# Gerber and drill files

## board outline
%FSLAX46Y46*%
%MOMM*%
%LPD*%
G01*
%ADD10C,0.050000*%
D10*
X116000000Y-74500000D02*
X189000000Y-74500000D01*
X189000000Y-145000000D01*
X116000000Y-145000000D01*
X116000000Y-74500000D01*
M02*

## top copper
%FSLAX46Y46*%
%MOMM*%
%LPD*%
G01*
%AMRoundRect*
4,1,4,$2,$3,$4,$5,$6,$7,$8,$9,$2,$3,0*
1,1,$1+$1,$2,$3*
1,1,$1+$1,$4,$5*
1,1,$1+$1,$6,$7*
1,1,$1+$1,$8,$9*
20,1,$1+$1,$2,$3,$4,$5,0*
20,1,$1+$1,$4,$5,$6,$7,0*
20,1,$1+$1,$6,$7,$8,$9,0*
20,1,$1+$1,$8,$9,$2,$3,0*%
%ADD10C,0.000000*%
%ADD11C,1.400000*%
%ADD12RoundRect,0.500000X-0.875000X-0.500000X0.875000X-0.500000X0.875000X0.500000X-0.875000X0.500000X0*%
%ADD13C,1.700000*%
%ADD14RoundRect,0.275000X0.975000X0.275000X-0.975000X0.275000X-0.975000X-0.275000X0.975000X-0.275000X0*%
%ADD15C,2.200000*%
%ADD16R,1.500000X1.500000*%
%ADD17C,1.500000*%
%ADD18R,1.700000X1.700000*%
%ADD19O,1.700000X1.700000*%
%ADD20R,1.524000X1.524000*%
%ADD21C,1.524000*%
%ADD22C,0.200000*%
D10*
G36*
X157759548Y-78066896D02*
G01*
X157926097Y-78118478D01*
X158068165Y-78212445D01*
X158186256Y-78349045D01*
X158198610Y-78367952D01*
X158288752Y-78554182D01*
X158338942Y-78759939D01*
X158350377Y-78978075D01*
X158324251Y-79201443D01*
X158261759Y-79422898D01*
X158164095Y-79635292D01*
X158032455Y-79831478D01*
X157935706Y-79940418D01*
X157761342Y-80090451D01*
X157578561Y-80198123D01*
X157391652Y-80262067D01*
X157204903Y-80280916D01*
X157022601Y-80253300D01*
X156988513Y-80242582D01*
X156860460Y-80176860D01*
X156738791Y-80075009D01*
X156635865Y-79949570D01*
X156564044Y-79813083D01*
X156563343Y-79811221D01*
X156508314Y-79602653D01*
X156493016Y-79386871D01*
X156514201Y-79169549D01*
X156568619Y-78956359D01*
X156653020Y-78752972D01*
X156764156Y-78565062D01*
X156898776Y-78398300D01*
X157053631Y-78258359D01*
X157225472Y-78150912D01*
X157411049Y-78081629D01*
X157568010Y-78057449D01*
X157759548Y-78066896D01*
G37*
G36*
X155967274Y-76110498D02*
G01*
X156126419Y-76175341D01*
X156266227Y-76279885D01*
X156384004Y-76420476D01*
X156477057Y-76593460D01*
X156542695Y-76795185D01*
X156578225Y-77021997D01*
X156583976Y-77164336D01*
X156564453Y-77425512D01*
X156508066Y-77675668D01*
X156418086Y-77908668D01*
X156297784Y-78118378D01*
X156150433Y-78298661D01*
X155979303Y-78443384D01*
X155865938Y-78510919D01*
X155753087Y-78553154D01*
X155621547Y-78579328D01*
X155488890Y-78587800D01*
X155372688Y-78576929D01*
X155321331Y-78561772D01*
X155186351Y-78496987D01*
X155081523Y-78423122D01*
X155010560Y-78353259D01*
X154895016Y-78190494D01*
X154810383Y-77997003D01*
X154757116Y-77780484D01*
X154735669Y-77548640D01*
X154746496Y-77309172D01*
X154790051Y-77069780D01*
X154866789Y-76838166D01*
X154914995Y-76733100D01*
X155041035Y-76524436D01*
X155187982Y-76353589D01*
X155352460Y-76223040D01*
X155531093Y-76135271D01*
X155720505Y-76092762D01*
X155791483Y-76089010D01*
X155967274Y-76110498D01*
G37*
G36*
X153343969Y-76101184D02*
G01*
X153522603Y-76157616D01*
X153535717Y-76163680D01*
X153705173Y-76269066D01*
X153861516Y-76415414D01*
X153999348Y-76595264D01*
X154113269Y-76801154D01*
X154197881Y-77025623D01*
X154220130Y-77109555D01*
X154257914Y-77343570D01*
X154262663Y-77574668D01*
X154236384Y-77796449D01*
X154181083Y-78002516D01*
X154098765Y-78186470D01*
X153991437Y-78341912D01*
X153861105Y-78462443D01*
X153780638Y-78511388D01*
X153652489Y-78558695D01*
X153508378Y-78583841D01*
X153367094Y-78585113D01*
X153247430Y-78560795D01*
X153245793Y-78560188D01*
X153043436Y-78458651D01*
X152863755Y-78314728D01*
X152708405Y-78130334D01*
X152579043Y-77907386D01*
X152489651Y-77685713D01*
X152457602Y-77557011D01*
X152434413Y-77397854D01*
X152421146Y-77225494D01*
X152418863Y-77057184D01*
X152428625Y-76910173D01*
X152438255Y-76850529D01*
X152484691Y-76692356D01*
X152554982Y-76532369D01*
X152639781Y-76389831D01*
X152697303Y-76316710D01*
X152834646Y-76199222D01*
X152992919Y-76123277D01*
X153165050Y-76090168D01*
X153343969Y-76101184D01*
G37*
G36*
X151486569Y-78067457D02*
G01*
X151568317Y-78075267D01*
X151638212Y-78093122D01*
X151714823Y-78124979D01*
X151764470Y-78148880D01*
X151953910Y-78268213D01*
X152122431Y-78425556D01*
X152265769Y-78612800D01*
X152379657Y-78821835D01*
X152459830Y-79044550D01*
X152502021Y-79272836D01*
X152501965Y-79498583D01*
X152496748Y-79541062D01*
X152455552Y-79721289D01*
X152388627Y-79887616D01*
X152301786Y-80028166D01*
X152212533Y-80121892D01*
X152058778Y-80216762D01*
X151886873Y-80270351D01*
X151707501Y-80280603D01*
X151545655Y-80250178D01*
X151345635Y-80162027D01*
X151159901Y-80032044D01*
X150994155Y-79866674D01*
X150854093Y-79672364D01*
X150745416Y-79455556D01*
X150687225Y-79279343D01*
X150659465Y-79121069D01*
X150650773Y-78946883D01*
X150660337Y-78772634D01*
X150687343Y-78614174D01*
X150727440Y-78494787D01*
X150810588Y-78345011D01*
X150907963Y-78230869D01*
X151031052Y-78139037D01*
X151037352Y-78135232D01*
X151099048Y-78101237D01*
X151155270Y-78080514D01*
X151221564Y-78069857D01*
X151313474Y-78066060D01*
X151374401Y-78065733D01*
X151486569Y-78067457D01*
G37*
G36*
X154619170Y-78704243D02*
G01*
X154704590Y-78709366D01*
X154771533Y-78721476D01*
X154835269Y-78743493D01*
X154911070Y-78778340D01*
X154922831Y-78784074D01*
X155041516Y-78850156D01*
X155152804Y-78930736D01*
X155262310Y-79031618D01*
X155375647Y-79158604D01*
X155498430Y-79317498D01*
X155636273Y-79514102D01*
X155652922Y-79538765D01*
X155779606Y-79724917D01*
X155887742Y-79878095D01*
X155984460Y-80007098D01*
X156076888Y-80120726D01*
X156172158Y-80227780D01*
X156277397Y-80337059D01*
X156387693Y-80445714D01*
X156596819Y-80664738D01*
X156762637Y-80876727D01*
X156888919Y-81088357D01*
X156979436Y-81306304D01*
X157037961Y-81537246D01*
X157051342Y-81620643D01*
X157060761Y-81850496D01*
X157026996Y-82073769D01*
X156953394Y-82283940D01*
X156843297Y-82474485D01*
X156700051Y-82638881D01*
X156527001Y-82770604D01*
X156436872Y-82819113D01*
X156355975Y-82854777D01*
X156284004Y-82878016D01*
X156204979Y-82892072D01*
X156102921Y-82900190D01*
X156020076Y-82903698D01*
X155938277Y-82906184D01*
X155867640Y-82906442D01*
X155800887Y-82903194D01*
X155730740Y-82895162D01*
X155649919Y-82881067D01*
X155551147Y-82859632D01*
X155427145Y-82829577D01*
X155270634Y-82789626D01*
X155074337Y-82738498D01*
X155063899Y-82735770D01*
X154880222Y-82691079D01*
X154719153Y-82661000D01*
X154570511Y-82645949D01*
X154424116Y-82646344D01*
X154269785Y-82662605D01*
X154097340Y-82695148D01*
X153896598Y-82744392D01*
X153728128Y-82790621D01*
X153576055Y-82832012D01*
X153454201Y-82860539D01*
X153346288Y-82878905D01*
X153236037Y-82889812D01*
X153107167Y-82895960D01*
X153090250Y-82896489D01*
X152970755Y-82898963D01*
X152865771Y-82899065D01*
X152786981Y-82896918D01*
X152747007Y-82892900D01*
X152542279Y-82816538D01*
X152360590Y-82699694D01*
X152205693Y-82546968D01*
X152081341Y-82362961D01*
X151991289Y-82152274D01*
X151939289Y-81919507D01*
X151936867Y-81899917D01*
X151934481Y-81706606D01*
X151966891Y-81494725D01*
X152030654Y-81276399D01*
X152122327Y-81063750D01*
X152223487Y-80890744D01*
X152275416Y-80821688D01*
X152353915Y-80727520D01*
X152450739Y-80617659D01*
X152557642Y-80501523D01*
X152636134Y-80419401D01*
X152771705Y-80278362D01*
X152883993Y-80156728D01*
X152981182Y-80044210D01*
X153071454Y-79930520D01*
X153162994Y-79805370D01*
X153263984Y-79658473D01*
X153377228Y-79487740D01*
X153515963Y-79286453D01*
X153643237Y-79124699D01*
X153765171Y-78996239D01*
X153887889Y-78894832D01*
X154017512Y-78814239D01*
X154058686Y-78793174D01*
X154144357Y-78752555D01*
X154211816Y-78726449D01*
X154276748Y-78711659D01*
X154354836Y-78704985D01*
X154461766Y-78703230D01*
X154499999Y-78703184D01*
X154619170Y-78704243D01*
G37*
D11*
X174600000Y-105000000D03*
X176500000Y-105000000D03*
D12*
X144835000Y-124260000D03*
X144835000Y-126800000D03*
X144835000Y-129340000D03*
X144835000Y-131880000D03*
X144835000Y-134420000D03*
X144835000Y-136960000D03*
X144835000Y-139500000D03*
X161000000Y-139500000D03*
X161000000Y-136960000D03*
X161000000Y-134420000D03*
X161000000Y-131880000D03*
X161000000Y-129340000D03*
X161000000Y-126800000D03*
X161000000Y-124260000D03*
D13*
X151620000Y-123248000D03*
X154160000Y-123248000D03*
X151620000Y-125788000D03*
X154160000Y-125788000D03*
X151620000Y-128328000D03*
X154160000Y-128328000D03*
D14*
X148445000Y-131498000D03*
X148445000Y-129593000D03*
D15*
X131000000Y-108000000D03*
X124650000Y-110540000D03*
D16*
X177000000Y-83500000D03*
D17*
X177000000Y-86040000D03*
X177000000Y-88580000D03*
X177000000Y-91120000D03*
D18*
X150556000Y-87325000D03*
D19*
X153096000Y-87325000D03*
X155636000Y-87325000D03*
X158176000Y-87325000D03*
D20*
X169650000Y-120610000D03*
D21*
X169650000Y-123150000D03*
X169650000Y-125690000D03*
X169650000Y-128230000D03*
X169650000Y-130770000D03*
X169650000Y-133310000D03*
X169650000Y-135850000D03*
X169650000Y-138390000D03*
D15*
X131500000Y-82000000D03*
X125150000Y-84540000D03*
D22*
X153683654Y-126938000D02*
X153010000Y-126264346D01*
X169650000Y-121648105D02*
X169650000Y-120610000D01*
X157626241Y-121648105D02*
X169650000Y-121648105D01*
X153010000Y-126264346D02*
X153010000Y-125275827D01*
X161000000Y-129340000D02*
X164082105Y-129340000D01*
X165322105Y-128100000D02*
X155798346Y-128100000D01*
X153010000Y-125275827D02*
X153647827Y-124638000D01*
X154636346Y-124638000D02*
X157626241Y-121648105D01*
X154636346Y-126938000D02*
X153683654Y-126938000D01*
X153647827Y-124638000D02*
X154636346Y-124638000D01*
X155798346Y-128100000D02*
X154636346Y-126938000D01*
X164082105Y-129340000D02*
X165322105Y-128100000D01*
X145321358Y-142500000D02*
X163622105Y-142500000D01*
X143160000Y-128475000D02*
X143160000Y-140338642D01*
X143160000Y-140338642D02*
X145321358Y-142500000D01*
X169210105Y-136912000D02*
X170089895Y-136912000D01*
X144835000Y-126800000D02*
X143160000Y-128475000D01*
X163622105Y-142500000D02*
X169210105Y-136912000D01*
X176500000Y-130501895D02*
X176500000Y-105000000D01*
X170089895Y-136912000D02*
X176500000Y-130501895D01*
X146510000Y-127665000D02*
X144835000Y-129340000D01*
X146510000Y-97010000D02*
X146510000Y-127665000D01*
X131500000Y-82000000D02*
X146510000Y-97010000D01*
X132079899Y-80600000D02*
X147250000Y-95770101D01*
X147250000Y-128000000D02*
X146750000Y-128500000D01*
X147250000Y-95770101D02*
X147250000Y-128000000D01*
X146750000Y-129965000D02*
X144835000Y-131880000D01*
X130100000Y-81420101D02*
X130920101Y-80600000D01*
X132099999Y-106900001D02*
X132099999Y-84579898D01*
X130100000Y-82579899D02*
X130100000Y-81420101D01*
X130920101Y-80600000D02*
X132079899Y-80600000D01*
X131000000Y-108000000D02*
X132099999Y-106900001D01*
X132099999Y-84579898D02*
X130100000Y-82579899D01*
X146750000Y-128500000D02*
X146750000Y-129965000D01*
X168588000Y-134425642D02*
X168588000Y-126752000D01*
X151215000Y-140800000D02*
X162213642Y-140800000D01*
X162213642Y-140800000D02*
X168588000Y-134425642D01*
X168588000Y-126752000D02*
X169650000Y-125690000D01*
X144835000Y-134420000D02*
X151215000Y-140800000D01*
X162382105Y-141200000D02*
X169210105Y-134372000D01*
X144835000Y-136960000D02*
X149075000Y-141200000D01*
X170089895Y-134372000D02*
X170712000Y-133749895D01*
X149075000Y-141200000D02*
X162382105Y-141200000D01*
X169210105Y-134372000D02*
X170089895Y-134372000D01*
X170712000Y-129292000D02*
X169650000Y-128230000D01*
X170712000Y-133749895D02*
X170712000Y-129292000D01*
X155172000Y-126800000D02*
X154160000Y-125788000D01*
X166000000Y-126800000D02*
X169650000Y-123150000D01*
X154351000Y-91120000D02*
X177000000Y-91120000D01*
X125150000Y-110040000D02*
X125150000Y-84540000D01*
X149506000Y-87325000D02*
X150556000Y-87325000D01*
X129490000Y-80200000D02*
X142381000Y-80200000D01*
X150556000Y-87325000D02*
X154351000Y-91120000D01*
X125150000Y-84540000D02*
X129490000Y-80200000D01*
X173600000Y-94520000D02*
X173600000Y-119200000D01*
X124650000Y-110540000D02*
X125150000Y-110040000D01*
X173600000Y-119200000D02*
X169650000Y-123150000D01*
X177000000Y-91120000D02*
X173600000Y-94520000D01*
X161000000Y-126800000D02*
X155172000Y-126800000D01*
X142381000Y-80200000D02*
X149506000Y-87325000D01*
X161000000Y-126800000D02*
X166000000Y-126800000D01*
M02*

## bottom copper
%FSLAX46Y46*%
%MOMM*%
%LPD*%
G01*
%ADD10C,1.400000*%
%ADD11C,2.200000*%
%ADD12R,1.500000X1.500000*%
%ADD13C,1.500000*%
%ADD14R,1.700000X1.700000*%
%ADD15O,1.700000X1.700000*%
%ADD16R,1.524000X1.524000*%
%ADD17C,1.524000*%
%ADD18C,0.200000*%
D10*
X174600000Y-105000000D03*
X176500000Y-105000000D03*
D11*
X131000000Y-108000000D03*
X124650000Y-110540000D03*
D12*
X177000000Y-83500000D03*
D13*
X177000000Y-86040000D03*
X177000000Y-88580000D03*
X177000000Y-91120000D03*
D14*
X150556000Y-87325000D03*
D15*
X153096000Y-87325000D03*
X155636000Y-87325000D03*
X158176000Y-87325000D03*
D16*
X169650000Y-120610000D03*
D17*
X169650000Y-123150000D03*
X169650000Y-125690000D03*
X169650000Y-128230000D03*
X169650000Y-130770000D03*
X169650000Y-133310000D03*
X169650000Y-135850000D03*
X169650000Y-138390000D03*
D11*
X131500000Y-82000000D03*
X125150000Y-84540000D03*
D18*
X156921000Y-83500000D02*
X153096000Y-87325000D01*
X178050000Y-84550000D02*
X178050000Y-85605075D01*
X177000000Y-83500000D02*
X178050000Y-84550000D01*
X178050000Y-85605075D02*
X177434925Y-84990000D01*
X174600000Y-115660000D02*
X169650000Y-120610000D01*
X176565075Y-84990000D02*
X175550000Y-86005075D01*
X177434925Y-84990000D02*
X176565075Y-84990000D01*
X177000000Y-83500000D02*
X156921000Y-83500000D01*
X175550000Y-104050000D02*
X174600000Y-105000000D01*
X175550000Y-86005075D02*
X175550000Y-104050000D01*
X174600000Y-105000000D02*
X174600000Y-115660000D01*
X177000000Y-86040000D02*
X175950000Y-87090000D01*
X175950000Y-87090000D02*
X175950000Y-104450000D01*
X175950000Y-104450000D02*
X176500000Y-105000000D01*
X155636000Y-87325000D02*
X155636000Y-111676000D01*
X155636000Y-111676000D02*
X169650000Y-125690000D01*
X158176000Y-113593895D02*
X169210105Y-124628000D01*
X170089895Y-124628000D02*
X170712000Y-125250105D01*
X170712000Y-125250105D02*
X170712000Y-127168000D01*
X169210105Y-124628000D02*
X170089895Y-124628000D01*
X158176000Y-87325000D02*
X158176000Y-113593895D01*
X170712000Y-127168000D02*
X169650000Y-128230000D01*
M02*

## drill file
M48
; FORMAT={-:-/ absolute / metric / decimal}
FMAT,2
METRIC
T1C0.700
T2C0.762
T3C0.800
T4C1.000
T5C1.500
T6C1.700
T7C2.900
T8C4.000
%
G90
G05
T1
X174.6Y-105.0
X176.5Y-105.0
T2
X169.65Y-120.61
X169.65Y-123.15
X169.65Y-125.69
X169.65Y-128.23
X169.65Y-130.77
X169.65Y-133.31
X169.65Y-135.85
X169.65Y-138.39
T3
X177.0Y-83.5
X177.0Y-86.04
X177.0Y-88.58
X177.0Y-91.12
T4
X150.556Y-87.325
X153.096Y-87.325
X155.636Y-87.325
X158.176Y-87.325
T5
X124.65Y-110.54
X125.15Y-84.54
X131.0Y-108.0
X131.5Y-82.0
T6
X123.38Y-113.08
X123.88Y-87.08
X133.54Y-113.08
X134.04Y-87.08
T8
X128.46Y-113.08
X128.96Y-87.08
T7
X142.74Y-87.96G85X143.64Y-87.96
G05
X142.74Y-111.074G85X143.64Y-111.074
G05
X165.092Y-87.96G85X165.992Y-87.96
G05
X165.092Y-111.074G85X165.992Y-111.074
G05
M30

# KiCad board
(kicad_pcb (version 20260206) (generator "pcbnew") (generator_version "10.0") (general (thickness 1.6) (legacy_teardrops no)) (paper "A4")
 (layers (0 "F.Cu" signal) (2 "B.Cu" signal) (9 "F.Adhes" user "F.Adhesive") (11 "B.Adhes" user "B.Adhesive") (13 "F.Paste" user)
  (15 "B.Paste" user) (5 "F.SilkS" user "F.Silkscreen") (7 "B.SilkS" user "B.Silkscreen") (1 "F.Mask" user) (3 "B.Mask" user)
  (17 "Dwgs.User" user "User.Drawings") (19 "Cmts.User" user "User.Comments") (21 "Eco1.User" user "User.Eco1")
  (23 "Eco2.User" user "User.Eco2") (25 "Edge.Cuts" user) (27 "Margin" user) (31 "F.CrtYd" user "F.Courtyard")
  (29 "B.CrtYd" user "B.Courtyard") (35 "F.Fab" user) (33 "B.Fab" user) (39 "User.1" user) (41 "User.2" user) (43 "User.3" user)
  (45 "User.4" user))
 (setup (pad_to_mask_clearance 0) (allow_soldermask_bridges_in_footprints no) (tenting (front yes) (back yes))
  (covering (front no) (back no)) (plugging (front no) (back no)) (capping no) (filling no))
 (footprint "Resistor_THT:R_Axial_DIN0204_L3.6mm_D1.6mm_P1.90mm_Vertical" (layer "F.Cu") (at 174.6 105)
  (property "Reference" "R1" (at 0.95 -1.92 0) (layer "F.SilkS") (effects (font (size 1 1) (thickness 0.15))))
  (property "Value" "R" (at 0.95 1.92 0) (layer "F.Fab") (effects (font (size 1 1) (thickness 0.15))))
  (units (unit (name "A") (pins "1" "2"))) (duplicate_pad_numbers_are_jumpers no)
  (pad "1" thru_hole circle (at 0 0) (size 1.4 1.4) (drill 0.7) (layers "*.Cu" "*.Mask") (remove_unused_layers no) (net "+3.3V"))
  (pad "2" thru_hole circle (at 1.9 0) (size 1.4 1.4) (drill 0.7) (layers "*.Cu" "*.Mask") (remove_unused_layers no) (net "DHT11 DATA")))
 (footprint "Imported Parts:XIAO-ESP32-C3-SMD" (layer "F.Cu") (at 144 142.38)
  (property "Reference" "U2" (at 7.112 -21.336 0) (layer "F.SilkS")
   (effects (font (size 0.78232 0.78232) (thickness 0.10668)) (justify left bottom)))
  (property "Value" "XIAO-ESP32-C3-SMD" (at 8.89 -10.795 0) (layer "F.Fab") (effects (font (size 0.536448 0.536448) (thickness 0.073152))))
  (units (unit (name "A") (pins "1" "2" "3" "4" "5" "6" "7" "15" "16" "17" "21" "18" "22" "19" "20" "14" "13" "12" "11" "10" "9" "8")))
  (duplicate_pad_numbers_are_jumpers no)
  (pad "1" smd roundrect (at 0.835 -18.12) (size 2.75 2) (layers "F.Cu" "F.Mask" "F.Paste") (roundrect_rratio 0.25)
   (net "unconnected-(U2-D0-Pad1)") (solder_mask_margin 0.0508) (thermal_bridge_angle 45))
  (pad "2" smd roundrect (at 0.835 -15.58) (size 2.75 2) (layers "F.Cu" "F.Mask" "F.Paste") (roundrect_rratio 0.25) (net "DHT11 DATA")
   (solder_mask_margin 0.0508) (thermal_bridge_angle 45))
  (pad "3" smd roundrect (at 0.835 -13.04) (size 2.75 2) (layers "F.Cu" "F.Mask" "F.Paste") (roundrect_rratio 0.25) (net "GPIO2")
   (solder_mask_margin 0.0508) (thermal_bridge_angle 45))
  (pad "4" smd roundrect (at 0.835 -10.5) (size 2.75 2) (layers "F.Cu" "F.Mask" "F.Paste") (roundrect_rratio 0.25) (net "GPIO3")
   (solder_mask_margin 0.0508) (thermal_bridge_angle 45))
  (pad "5" smd roundrect (at 0.835 -7.96) (size 2.75 2) (layers "F.Cu" "F.Mask" "F.Paste") (roundrect_rratio 0.25) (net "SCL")
   (solder_mask_margin 0.0508) (thermal_bridge_angle 45))
  (pad "6" smd roundrect (at 0.835 -5.42) (size 2.75 2) (layers "F.Cu" "F.Mask" "F.Paste") (roundrect_rratio 0.25) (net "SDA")
   (solder_mask_margin 0.0508) (thermal_bridge_angle 45))
  (pad "7" smd roundrect (at 0.835 -2.88) (size 2.75 2) (layers "F.Cu" "F.Mask" "F.Paste") (roundrect_rratio 0.25)
   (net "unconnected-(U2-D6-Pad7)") (solder_mask_margin 0.0508) (thermal_bridge_angle 45))
  (pad "8" smd roundrect (at 17 -2.88) (size 2.75 2) (layers "F.Cu" "F.Mask" "F.Paste") (roundrect_rratio 0.25)
   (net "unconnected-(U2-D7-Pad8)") (solder_mask_margin 0.0508) (thermal_bridge_angle 45))
  (pad "9" smd roundrect (at 17 -5.42) (size 2.75 2) (layers "F.Cu" "F.Mask" "F.Paste") (roundrect_rratio 0.25)
   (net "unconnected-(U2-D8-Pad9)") (solder_mask_margin 0.0508) (thermal_bridge_angle 45))
  (pad "10" smd roundrect (at 17 -7.96) (size 2.75 2) (layers "F.Cu" "F.Mask" "F.Paste") (roundrect_rratio 0.25)
   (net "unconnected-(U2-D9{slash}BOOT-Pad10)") (solder_mask_margin 0.0508) (thermal_bridge_angle 45))
  (pad "11" smd roundrect (at 17 -10.5) (size 2.75 2) (layers "F.Cu" "F.Mask" "F.Paste") (roundrect_rratio 0.25)
   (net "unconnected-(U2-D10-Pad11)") (solder_mask_margin 0.0508) (thermal_bridge_angle 45))
  (pad "12" smd roundrect (at 17 -13.04) (size 2.75 2) (layers "F.Cu" "F.Mask" "F.Paste") (roundrect_rratio 0.25) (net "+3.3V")
   (solder_mask_margin 0.0508) (thermal_bridge_angle 45))
  (pad "13" smd roundrect (at 17 -15.58) (size 2.75 2) (layers "F.Cu" "F.Mask" "F.Paste") (roundrect_rratio 0.25) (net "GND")
   (solder_mask_margin 0.0508) (thermal_bridge_angle 45))
  (pad "14" smd roundrect (at 17 -18.12) (size 2.75 2) (layers "F.Cu" "F.Mask" "F.Paste") (roundrect_rratio 0.25) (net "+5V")
   (solder_mask_margin 0.0508) (thermal_bridge_angle 45))
  (pad "15" smd circle (at 7.62 -19.132) (size 1.7 1.7) (layers "F.Cu" "F.Mask" "F.Paste") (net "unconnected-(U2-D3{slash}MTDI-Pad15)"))
  (pad "16" smd circle (at 10.16 -19.132) (size 1.7 1.7) (layers "F.Cu" "F.Mask" "F.Paste") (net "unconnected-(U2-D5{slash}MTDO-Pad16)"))
  (pad "17" smd circle (at 7.62 -16.592) (size 1.7 1.7) (layers "F.Cu" "F.Mask" "F.Paste") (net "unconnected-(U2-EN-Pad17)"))
  (pad "18" smd circle (at 10.16 -16.592) (size 1.7 1.7) (layers "F.Cu" "F.Mask" "F.Paste") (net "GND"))
  (pad "19" smd circle (at 7.62 -14.052) (size 1.7 1.7) (layers "F.Cu" "F.Mask" "F.Paste") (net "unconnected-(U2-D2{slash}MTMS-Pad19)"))
  (pad "20" smd circle (at 10.16 -14.052) (size 1.7 1.7) (layers "F.Cu" "F.Mask" "F.Paste") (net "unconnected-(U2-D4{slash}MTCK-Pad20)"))
  (pad "21" smd roundrect (at 4.445 -10.882 180) (size 2.5 1.1) (layers "F.Cu" "F.Mask" "F.Paste") (roundrect_rratio 0.25)
   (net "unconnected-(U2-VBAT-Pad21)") (thermal_bridge_angle 45))
  (pad "22" smd roundrect (at 4.445 -12.787 180) (size 2.5 1.1) (layers "F.Cu" "F.Mask" "F.Paste") (roundrect_rratio 0.25)
   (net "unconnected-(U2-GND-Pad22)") (thermal_bridge_angle 45)))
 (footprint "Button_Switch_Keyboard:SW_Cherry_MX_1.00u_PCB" (layer "F.Cu") (at 131 108)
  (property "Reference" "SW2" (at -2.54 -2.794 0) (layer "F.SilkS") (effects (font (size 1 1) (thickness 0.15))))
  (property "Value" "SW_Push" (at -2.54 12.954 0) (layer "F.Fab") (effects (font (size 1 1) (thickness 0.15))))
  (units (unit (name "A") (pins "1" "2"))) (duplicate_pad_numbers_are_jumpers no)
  (pad "" np_thru_hole circle (at -7.62 5.08) (size 1.7 1.7) (drill 1.7) (layers "*.Cu" "*.Mask"))
  (pad "" np_thru_hole circle (at -2.54 5.08) (size 4 4) (drill 4) (layers "*.Cu" "*.Mask"))
  (pad "" np_thru_hole circle (at 2.54 5.08) (size 1.7 1.7) (drill 1.7) (layers "*.Cu" "*.Mask"))
  (pad "1" thru_hole circle (at 0 0) (size 2.2 2.2) (drill 1.5) (layers "*.Cu" "*.Mask") (remove_unused_layers no) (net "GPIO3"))
  (pad "2" thru_hole circle (at -6.35 2.54) (size 2.2 2.2) (drill 1.5) (layers "*.Cu" "*.Mask") (remove_unused_layers no) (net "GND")))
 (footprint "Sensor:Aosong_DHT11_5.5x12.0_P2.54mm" (layer "F.Cu") (at 177 83.5)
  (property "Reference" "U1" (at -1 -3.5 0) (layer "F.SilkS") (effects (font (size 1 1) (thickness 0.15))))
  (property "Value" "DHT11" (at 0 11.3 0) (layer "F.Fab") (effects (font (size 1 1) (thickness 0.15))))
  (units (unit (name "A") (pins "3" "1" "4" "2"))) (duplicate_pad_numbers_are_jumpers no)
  (pad "1" thru_hole rect (at 0 0) (size 1.5 1.5) (drill 0.8) (layers "*.Cu" "*.Mask") (remove_unused_layers no) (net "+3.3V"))
  (pad "2" thru_hole circle (at 0 2.54) (size 1.5 1.5) (drill 0.8) (layers "*.Cu" "*.Mask") (remove_unused_layers no) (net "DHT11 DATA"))
  (pad "3" thru_hole circle (at 0 5.08) (size 1.5 1.5) (drill 0.8) (layers "*.Cu" "*.Mask") (remove_unused_layers no)
   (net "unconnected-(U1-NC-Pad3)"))
  (pad "4" thru_hole circle (at 0 7.62) (size 1.5 1.5) (drill 0.8) (layers "*.Cu" "*.Mask") (remove_unused_layers no) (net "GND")))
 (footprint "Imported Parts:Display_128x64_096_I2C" (layer "F.Cu") (at 154.366 87.325)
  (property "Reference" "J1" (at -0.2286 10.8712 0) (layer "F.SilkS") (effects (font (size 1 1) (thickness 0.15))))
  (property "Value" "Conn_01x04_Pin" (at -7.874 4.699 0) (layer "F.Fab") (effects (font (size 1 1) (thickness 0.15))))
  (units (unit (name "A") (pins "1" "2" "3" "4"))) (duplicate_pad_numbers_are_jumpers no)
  (pad "" np_thru_hole oval (at -11.176 0.635) (size 3.8 2.9) (drill oval 3.8 2.9) (layers "*.Cu" "*.Mask"))
  (pad "" np_thru_hole oval (at -11.176 23.749) (size 3.8 2.9) (drill oval 3.8 2.9) (layers "*.Cu" "*.Mask"))
  (pad "" np_thru_hole oval (at 11.176 0.635) (size 3.8 2.9) (drill oval 3.8 2.9) (layers "*.Cu" "*.Mask"))
  (pad "" np_thru_hole oval (at 11.176 23.749) (size 3.8 2.9) (drill oval 3.8 2.9) (layers "*.Cu" "*.Mask"))
  (pad "1" thru_hole rect (at -3.81 0 90) (size 1.7 1.7) (drill 1) (layers "*.Cu" "*.Mask") (remove_unused_layers no) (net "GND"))
  (pad "2" thru_hole oval (at -1.27 0 90) (size 1.7 1.7) (drill 1) (layers "*.Cu" "*.Mask") (remove_unused_layers no) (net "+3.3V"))
  (pad "3" thru_hole oval (at 1.27 0 90) (size 1.7 1.7) (drill 1) (layers "*.Cu" "*.Mask") (remove_unused_layers no) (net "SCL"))
  (pad "4" thru_hole oval (at 3.81 0 90) (size 1.7 1.7) (drill 1) (layers "*.Cu" "*.Mask") (remove_unused_layers no) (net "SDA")))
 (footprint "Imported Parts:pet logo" (layer "F.Cu") (at 154.5 79.5)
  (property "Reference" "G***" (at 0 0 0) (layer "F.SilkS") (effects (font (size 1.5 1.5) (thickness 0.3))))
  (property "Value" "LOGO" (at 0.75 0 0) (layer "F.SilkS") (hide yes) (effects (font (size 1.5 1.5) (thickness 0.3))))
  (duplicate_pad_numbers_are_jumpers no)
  (fp_poly
   (pts (xy 3.259548 -1.433104) (xy 3.426097 -1.381522) (xy 3.568165 -1.287555) (xy 3.686256 -1.150955) (xy 3.69861 -1.132048)
    (xy 3.788752 -0.945818) (xy 3.838942 -0.740061) (xy 3.850377 -0.521925) (xy 3.824251 -0.298557) (xy 3.761759 -0.077102)
    (xy 3.664095 0.135292) (xy 3.532455 0.331478) (xy 3.435706 0.440418) (xy 3.261342 0.590451) (xy 3.078561 0.698123)
    (xy 2.891652 0.762067) (xy 2.704903 0.780916) (xy 2.522601 0.7533) (xy 2.488513 0.742582) (xy 2.36046 0.67686) (xy 2.238791 0.575009)
    (xy 2.135865 0.44957) (xy 2.064044 0.313083) (xy 2.063343 0.311221) (xy 2.008314 0.102653) (xy 1.993016 -0.113129)
    (xy 2.014201 -0.330451) (xy 2.068619 -0.543641) (xy 2.15302 -0.747028) (xy 2.264156 -0.934938) (xy 2.398776 -1.1017)
    (xy 2.553631 -1.241641) (xy 2.725472 -1.349088) (xy 2.911049 -1.418371) (xy 3.06801 -1.442551))
   (stroke (width 0) (type solid)) (fill yes) (layer "F.Cu"))
  (fp_poly
   (pts (xy 1.467274 -3.389502) (xy 1.626419 -3.324659) (xy 1.766227 -3.220115) (xy 1.884004 -3.079524) (xy 1.977057 -2.90654)
    (xy 2.042695 -2.704815) (xy 2.078225 -2.478003) (xy 2.083976 -2.335664) (xy 2.064453 -2.074488) (xy 2.008066 -1.824332)
    (xy 1.918086 -1.591332) (xy 1.797784 -1.381622) (xy 1.650433 -1.201339) (xy 1.479303 -1.056616) (xy 1.365938 -0.989081)
    (xy 1.253087 -0.946846) (xy 1.121547 -0.920672) (xy 0.98889 -0.9122) (xy 0.872688 -0.923071) (xy 0.821331 -0.938228)
    (xy 0.686351 -1.003013) (xy 0.581523 -1.076878) (xy 0.51056 -1.146741) (xy 0.395016 -1.309506) (xy 0.310383 -1.502997)
    (xy 0.257116 -1.719516) (xy 0.235669 -1.95136) (xy 0.246496 -2.190828) (xy 0.290051 -2.43022) (xy 0.366789 -2.661834)
    (xy 0.414995 -2.7669) (xy 0.541035 -2.975564) (xy 0.687982 -3.146411) (xy 0.85246 -3.27696) (xy 1.031093 -3.364729)
    (xy 1.220505 -3.407238) (xy 1.291483 -3.41099))
   (stroke (width 0) (type solid)) (fill yes) (layer "F.Cu"))
  (fp_poly
   (pts (xy -1.156031 -3.398816) (xy -0.977397 -3.342384) (xy -0.964283 -3.33632) (xy -0.794827 -3.230934) (xy -0.638484 -3.084586)
    (xy -0.500652 -2.904736) (xy -0.386731 -2.698846) (xy -0.302119 -2.474377) (xy -0.27987 -2.390445) (xy -0.242086 -2.15643)
    (xy -0.237337 -1.925332) (xy -0.263616 -1.703551) (xy -0.318917 -1.497484) (xy -0.401235 -1.31353) (xy -0.508563 -1.158088)
    (xy -0.638895 -1.037557) (xy -0.719362 -0.988612) (xy -0.847511 -0.941305) (xy -0.991622 -0.916159) (xy -1.132906 -0.914887)
    (xy -1.25257 -0.939205) (xy -1.254207 -0.939812) (xy -1.456564 -1.041349) (xy -1.636245 -1.185272) (xy -1.791595 -1.369666)
    (xy -1.920957 -1.592614) (xy -2.010349 -1.814287) (xy -2.042398 -1.942989) (xy -2.065587 -2.102146) (xy -2.078854 -2.274506)
    (xy -2.081137 -2.442816) (xy -2.071375 -2.589827) (xy -2.061745 -2.649471) (xy -2.015309 -2.807644) (xy -1.945018 -2.967631)
    (xy -1.860219 -3.110169) (xy -1.802697 -3.18329) (xy -1.665354 -3.300778) (xy -1.507081 -3.376723) (xy -1.33495 -3.409832))
   (stroke (width 0) (type solid)) (fill yes) (layer "F.Cu"))
  (fp_poly
   (pts (xy -3.013431 -1.432543) (xy -2.931683 -1.424733) (xy -2.861788 -1.406878) (xy -2.785177 -1.375021) (xy -2.73553 -1.35112)
    (xy -2.54609 -1.231787) (xy -2.377569 -1.074444) (xy -2.234231 -0.8872) (xy -2.120343 -0.678165) (xy -2.04017 -0.45545)
    (xy -1.997979 -0.227164) (xy -1.998035 -0.001417) (xy -2.003252 0.041062) (xy -2.044448 0.221289) (xy -2.111373 0.387616)
    (xy -2.198214 0.528166) (xy -2.287467 0.621892) (xy -2.441222 0.716762) (xy -2.613127 0.770351) (xy -2.792499 0.780603)
    (xy -2.954345 0.750178) (xy -3.154365 0.662027) (xy -3.340099 0.532044) (xy -3.505845 0.366674) (xy -3.645907 0.172364)
    (xy -3.754584 -0.044444) (xy -3.812775 -0.220657) (xy -3.840535 -0.378931) (xy -3.849227 -0.553117) (xy -3.839663 -0.727366)
    (xy -3.812657 -0.885826) (xy -3.77256 -1.005213) (xy -3.689412 -1.154989) (xy -3.592037 -1.269131) (xy -3.468948 -1.360963)
    (xy -3.462648 -1.364768) (xy -3.400952 -1.398763) (xy -3.34473 -1.419486) (xy -3.278436 -1.430143) (xy -3.186526 -1.43394)
    (xy -3.125599 -1.434267))
   (stroke (width 0) (type solid)) (fill yes) (layer "F.Cu"))
  (fp_poly
   (pts (xy 0.11917 -0.795757) (xy 0.20459 -0.790634) (xy 0.271533 -0.778524) (xy 0.335269 -0.756507) (xy 0.41107 -0.72166)
    (xy 0.422831 -0.715926) (xy 0.541516 -0.649844) (xy 0.652804 -0.569264) (xy 0.76231 -0.468382) (xy 0.875647 -0.341396)
    (xy 0.99843 -0.182502) (xy 1.136273 0.014102) (xy 1.152922 0.038765) (xy 1.279606 0.224917) (xy 1.387742 0.378095) (xy 1.48446 0.507098)
    (xy 1.576888 0.620726) (xy 1.672158 0.72778) (xy 1.777397 0.837059) (xy 1.887693 0.945714) (xy 2.096819 1.164738) (xy 2.262637 1.376727)
    (xy 2.388919 1.588357) (xy 2.479436 1.806304) (xy 2.537961 2.037246) (xy 2.551342 2.120643) (xy 2.560761 2.350496)
    (xy 2.526996 2.573769) (xy 2.453394 2.78394) (xy 2.343297 2.974485) (xy 2.200051 3.138881) (xy 2.027001 3.270604) (xy 1.936872 3.319113)
    (xy 1.855975 3.354777) (xy 1.784004 3.378016) (xy 1.704979 3.392072) (xy 1.602921 3.40019) (xy 1.520076 3.403698) (xy 1.438277 3.406184)
    (xy 1.36764 3.406442) (xy 1.300887 3.403194) (xy 1.23074 3.395162) (xy 1.149919 3.381067) (xy 1.051147 3.359632) (xy 0.927145 3.329577)
    (xy 0.770634 3.289626) (xy 0.574337 3.238498) (xy 0.563899 3.23577) (xy 0.380222 3.191079) (xy 0.219153 3.161) (xy 0.070511 3.145949)
    (xy -0.075884 3.146344) (xy -0.230215 3.162605) (xy -0.40266 3.195148) (xy -0.603402 3.244392) (xy -0.771872 3.290621)
    (xy -0.923945 3.332012) (xy -1.045799 3.360539) (xy -1.153712 3.378905) (xy -1.263963 3.389812) (xy -1.392833 3.39596)
    (xy -1.40975 3.396489) (xy -1.529245 3.398963) (xy -1.634229 3.399065) (xy -1.713019 3.396918) (xy -1.752993 3.3929)
    (xy -1.957721 3.316538) (xy -2.13941 3.199694) (xy -2.294307 3.046968) (xy -2.418659 2.862961) (xy -2.508711 2.652274)
    (xy -2.560711 2.419507) (xy -2.563133 2.399917) (xy -2.565519 2.206606) (xy -2.533109 1.994725) (xy -2.469346 1.776399)
    (xy -2.377673 1.56375) (xy -2.276513 1.390744) (xy -2.224584 1.321688) (xy -2.146085 1.22752) (xy -2.049261 1.117659)
    (xy -1.942358 1.001523) (xy -1.863866 0.919401) (xy -1.728295 0.778362) (xy -1.616007 0.656728) (xy -1.518818 0.54421)
    (xy -1.428546 0.43052) (xy -1.337006 0.30537) (xy -1.236016 0.158473) (xy -1.122772 -0.01226) (xy -0.984037 -0.213547)
    (xy -0.856763 -0.375301) (xy -0.734829 -0.503761) (xy -0.612111 -0.605168) (xy -0.482488 -0.685761) (xy -0.441314 -0.706826)
    (xy -0.355643 -0.747445) (xy -0.288184 -0.773551) (xy -0.223252 -0.788341) (xy -0.145164 -0.795015) (xy -0.038234 -0.79677)
    (xy -0.000001 -0.796816))
   (stroke (width 0) (type solid)) (fill yes) (layer "F.Cu")))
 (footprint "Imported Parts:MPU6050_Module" (layer "F.Cu") (at 169.65 120.61)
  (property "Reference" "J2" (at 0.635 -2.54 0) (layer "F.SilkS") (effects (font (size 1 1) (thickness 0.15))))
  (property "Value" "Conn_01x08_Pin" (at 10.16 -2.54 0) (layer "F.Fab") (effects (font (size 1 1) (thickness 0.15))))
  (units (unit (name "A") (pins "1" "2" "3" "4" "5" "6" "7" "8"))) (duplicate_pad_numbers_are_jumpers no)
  (pad "1" thru_hole rect (at 0 0) (size 1.524 1.524) (drill 0.762) (layers "*.Cu" "*.Mask") (remove_unused_layers no) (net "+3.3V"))
  (pad "2" thru_hole circle (at 0 2.54) (size 1.524 1.524) (drill 0.762) (layers "*.Cu" "*.Mask") (remove_unused_layers no) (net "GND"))
  (pad "3" thru_hole circle (at 0 5.08) (size 1.524 1.524) (drill 0.762) (layers "*.Cu" "*.Mask") (remove_unused_layers no) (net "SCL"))
  (pad "4" thru_hole circle (at 0 7.62) (size 1.524 1.524) (drill 0.762) (layers "*.Cu" "*.Mask") (remove_unused_layers no) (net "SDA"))
  (pad "5" thru_hole circle (at 0 10.16) (size 1.524 1.524) (drill 0.762) (layers "*.Cu" "*.Mask") (remove_unused_layers no)
   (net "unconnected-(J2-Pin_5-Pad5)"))
  (pad "6" thru_hole circle (at 0 12.7) (size 1.524 1.524) (drill 0.762) (layers "*.Cu" "*.Mask") (remove_unused_layers no)
   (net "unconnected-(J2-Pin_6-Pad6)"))
  (pad "7" thru_hole circle (at 0 15.24) (size 1.524 1.524) (drill 0.762) (layers "*.Cu" "*.Mask") (remove_unused_layers no)
   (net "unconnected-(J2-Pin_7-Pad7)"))
  (pad "8" thru_hole circle (at 0 17.78) (size 1.524 1.524) (drill 0.762) (layers "*.Cu" "*.Mask") (remove_unused_layers no)
   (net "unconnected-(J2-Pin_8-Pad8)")))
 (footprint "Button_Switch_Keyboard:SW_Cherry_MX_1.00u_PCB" (layer "F.Cu") (at 131.5 82)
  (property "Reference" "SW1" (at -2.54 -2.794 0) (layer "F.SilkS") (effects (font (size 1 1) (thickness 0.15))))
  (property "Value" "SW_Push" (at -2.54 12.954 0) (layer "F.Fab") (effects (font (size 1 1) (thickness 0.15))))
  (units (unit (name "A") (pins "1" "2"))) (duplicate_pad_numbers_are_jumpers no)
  (pad "" np_thru_hole circle (at -7.62 5.08) (size 1.7 1.7) (drill 1.7) (layers "*.Cu" "*.Mask"))
  (pad "" np_thru_hole circle (at -2.54 5.08) (size 4 4) (drill 4) (layers "*.Cu" "*.Mask"))
  (pad "" np_thru_hole circle (at 2.54 5.08) (size 1.7 1.7) (drill 1.7) (layers "*.Cu" "*.Mask"))
  (pad "1" thru_hole circle (at 0 0) (size 2.2 2.2) (drill 1.5) (layers "*.Cu" "*.Mask") (remove_unused_layers no) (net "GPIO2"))
  (pad "2" thru_hole circle (at -6.35 2.54) (size 2.2 2.2) (drill 1.5) (layers "*.Cu" "*.Mask") (remove_unused_layers no) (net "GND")))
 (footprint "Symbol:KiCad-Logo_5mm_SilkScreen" (layer "F.Cu") (at 130 134)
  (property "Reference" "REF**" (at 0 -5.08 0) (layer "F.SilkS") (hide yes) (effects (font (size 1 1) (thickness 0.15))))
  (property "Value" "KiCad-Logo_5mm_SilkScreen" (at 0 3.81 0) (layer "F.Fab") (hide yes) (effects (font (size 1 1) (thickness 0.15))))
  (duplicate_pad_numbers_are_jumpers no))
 (gr_rect (start 116 74.5) (end 189 145) (stroke (width 0.05) (type default)) (fill no) (layer "Edge.Cuts"))
 (segment (start 153.683654 126.938) (end 153.01 126.264346) (width 0.2) (layer "F.Cu") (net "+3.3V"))
 (segment (start 169.65 121.648105) (end 169.65 120.61) (width 0.2) (layer "F.Cu") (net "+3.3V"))
 (segment (start 157.626241 121.648105) (end 169.65 121.648105) (width 0.2) (layer "F.Cu") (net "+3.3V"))
 (segment (start 153.01 126.264346) (end 153.01 125.275827) (width 0.2) (layer "F.Cu") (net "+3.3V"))
 (segment (start 161 129.34) (end 164.082105 129.34) (width 0.2) (layer "F.Cu") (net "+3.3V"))
 (segment (start 165.322105 128.1) (end 155.798346 128.1) (width 0.2) (layer "F.Cu") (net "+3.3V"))
 (segment (start 153.01 125.275827) (end 153.647827 124.638) (width 0.2) (layer "F.Cu") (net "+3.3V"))
 (segment (start 154.636346 124.638) (end 157.626241 121.648105) (width 0.2) (layer "F.Cu") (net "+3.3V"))
 (segment (start 154.636346 126.938) (end 153.683654 126.938) (width 0.2) (layer "F.Cu") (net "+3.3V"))
 (segment (start 153.647827 124.638) (end 154.636346 124.638) (width 0.2) (layer "F.Cu") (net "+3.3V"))
 (segment (start 155.798346 128.1) (end 154.636346 126.938) (width 0.2) (layer "F.Cu") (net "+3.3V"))
 (segment (start 164.082105 129.34) (end 165.322105 128.1) (width 0.2) (layer "F.Cu") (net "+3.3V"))
 (segment (start 156.921 83.5) (end 153.096 87.325) (width 0.2) (layer "B.Cu") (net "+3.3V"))
 (segment (start 178.05 84.55) (end 178.05 85.605075) (width 0.2) (layer "B.Cu") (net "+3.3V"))
 (segment (start 177 83.5) (end 178.05 84.55) (width 0.2) (layer "B.Cu") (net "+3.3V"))
 (segment (start 178.05 85.605075) (end 177.434925 84.99) (width 0.2) (layer "B.Cu") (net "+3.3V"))
 (segment (start 174.6 115.66) (end 169.65 120.61) (width 0.2) (layer "B.Cu") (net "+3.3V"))
 (segment (start 176.565075 84.99) (end 175.55 86.005075) (width 0.2) (layer "B.Cu") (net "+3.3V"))
 (segment (start 177.434925 84.99) (end 176.565075 84.99) (width 0.2) (layer "B.Cu") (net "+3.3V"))
 (segment (start 177 83.5) (end 156.921 83.5) (width 0.2) (layer "B.Cu") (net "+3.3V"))
 (segment (start 175.55 104.05) (end 174.6 105) (width 0.2) (layer "B.Cu") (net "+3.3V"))
 (segment (start 175.55 86.005075) (end 175.55 104.05) (width 0.2) (layer "B.Cu") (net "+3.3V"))
 (segment (start 174.6 105) (end 174.6 115.66) (width 0.2) (layer "B.Cu") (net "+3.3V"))
 (segment (start 145.321358 142.5) (end 163.622105 142.5) (width 0.2) (layer "F.Cu") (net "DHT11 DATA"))
 (segment (start 143.16 128.475) (end 143.16 140.338642) (width 0.2) (layer "F.Cu") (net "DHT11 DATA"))
 (segment (start 143.16 140.338642) (end 145.321358 142.5) (width 0.2) (layer "F.Cu") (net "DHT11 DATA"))
 (segment (start 169.210105 136.912) (end 170.089895 136.912) (width 0.2) (layer "F.Cu") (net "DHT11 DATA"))
 (segment (start 144.835 126.8) (end 143.16 128.475) (width 0.2) (layer "F.Cu") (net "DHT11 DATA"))
 (segment (start 163.622105 142.5) (end 169.210105 136.912) (width 0.2) (layer "F.Cu") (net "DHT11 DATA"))
 (segment (start 176.5 130.501895) (end 176.5 105) (width 0.2) (layer "F.Cu") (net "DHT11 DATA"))
 (segment (start 170.089895 136.912) (end 176.5 130.501895) (width 0.2) (layer "F.Cu") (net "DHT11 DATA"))
 (segment (start 177 86.04) (end 175.95 87.09) (width 0.2) (layer "B.Cu") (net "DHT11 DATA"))
 (segment (start 175.95 87.09) (end 175.95 104.45) (width 0.2) (layer "B.Cu") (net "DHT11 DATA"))
 (segment (start 175.95 104.45) (end 176.5 105) (width 0.2) (layer "B.Cu") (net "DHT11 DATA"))
 (segment (start 146.51 127.665) (end 144.835 129.34) (width 0.2) (layer "F.Cu") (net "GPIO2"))
 (segment (start 146.51 97.01) (end 146.51 127.665) (width 0.2) (layer "F.Cu") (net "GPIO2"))
 (segment (start 131.5 82) (end 146.51 97.01) (width 0.2) (layer "F.Cu") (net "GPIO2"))
 (segment (start 132.079899 80.6) (end 147.25 95.770101) (width 0.2) (layer "F.Cu") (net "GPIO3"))
 (segment (start 147.25 128) (end 146.75 128.5) (width 0.2) (layer "F.Cu") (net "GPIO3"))
 (segment (start 147.25 95.770101) (end 147.25 128) (width 0.2) (layer "F.Cu") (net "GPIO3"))
 (segment (start 146.75 129.965) (end 144.835 131.88) (width 0.2) (layer "F.Cu") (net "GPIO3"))
 (segment (start 130.1 81.420101) (end 130.920101 80.6) (width 0.2) (layer "F.Cu") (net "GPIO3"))
 (segment (start 132.099999 106.900001) (end 132.099999 84.579898) (width 0.2) (layer "F.Cu") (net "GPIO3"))
 (segment (start 130.1 82.579899) (end 130.1 81.420101) (width 0.2) (layer "F.Cu") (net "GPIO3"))
 (segment (start 130.920101 80.6) (end 132.079899 80.6) (width 0.2) (layer "F.Cu") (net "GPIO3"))
 (segment (start 131 108) (end 132.099999 106.900001) (width 0.2) (layer "F.Cu") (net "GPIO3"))
 (segment (start 132.099999 84.579898) (end 130.1 82.579899) (width 0.2) (layer "F.Cu") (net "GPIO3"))
 (segment (start 146.75 128.5) (end 146.75 129.965) (width 0.2) (layer "F.Cu") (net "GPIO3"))
 (segment (start 168.588 134.425642) (end 168.588 126.752) (width 0.2) (layer "F.Cu") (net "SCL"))
 (segment (start 151.215 140.8) (end 162.213642 140.8) (width 0.2) (layer "F.Cu") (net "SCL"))
 (segment (start 162.213642 140.8) (end 168.588 134.425642) (width 0.2) (layer "F.Cu") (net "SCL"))
 (segment (start 168.588 126.752) (end 169.65 125.69) (width 0.2) (layer "F.Cu") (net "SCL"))
 (segment (start 144.835 134.42) (end 151.215 140.8) (width 0.2) (layer "F.Cu") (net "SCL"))
 (segment (start 155.636 87.325) (end 155.636 111.676) (width 0.2) (layer "B.Cu") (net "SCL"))
 (segment (start 155.636 111.676) (end 169.65 125.69) (width 0.2) (layer "B.Cu") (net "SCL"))
 (segment (start 162.382105 141.2) (end 169.210105 134.372) (width 0.2) (layer "F.Cu") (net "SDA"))
 (segment (start 144.835 136.96) (end 149.075 141.2) (width 0.2) (layer "F.Cu") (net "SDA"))
 (segment (start 170.089895 134.372) (end 170.712 133.749895) (width 0.2) (layer "F.Cu") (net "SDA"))
 (segment (start 149.075 141.2) (end 162.382105 141.2) (width 0.2) (layer "F.Cu") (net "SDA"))
 (segment (start 169.210105 134.372) (end 170.089895 134.372) (width 0.2) (layer "F.Cu") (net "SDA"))
 (segment (start 170.712 129.292) (end 169.65 128.23) (width 0.2) (layer "F.Cu") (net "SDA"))
 (segment (start 170.712 133.749895) (end 170.712 129.292) (width 0.2) (layer "F.Cu") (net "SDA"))
 (segment (start 158.176 113.593895) (end 169.210105 124.628) (width 0.2) (layer "B.Cu") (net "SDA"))
 (segment (start 170.089895 124.628) (end 170.712 125.250105) (width 0.2) (layer "B.Cu") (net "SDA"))
 (segment (start 170.712 125.250105) (end 170.712 127.168) (width 0.2) (layer "B.Cu") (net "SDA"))
 (segment (start 169.210105 124.628) (end 170.089895 124.628) (width 0.2) (layer "B.Cu") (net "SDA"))
 (segment (start 158.176 87.325) (end 158.176 113.593895) (width 0.2) (layer "B.Cu") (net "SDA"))
 (segment (start 170.712 127.168) (end 169.65 128.23) (width 0.2) (layer "B.Cu") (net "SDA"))
 (segment (start 155.172 126.8) (end 154.16 125.788) (width 0.2) (layer "F.Cu") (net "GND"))
 (segment (start 166 126.8) (end 169.65 123.15) (width 0.2) (layer "F.Cu") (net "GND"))
 (segment (start 154.351 91.12) (end 177 91.12) (width 0.2) (layer "F.Cu") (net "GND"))
 (segment (start 125.15 110.04) (end 125.15 84.54) (width 0.2) (layer "F.Cu") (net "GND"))
 (segment (start 149.506 87.325) (end 150.556 87.325) (width 0.2) (layer "F.Cu") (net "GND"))
 (segment (start 129.49 80.2) (end 142.381 80.2) (width 0.2) (layer "F.Cu") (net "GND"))
 (segment (start 150.556 87.325) (end 154.351 91.12) (width 0.2) (layer "F.Cu") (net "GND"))
 (segment (start 125.15 84.54) (end 129.49 80.2) (width 0.2) (layer "F.Cu") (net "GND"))
 (segment (start 173.6 94.52) (end 173.6 119.2) (width 0.2) (layer "F.Cu") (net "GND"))
 (segment (start 124.65 110.54) (end 125.15 110.04) (width 0.2) (layer "F.Cu") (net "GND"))
 (segment (start 173.6 119.2) (end 169.65 123.15) (width 0.2) (layer "F.Cu") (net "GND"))
 (segment (start 177 91.12) (end 173.6 94.52) (width 0.2) (layer "F.Cu") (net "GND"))
 (segment (start 161 126.8) (end 155.172 126.8) (width 0.2) (layer "F.Cu") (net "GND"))
 (segment (start 142.381 80.2) (end 149.506 87.325) (width 0.2) (layer "F.Cu") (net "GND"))
 (segment (start 161 126.8) (end 166 126.8) (width 0.2) (layer "F.Cu") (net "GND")))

